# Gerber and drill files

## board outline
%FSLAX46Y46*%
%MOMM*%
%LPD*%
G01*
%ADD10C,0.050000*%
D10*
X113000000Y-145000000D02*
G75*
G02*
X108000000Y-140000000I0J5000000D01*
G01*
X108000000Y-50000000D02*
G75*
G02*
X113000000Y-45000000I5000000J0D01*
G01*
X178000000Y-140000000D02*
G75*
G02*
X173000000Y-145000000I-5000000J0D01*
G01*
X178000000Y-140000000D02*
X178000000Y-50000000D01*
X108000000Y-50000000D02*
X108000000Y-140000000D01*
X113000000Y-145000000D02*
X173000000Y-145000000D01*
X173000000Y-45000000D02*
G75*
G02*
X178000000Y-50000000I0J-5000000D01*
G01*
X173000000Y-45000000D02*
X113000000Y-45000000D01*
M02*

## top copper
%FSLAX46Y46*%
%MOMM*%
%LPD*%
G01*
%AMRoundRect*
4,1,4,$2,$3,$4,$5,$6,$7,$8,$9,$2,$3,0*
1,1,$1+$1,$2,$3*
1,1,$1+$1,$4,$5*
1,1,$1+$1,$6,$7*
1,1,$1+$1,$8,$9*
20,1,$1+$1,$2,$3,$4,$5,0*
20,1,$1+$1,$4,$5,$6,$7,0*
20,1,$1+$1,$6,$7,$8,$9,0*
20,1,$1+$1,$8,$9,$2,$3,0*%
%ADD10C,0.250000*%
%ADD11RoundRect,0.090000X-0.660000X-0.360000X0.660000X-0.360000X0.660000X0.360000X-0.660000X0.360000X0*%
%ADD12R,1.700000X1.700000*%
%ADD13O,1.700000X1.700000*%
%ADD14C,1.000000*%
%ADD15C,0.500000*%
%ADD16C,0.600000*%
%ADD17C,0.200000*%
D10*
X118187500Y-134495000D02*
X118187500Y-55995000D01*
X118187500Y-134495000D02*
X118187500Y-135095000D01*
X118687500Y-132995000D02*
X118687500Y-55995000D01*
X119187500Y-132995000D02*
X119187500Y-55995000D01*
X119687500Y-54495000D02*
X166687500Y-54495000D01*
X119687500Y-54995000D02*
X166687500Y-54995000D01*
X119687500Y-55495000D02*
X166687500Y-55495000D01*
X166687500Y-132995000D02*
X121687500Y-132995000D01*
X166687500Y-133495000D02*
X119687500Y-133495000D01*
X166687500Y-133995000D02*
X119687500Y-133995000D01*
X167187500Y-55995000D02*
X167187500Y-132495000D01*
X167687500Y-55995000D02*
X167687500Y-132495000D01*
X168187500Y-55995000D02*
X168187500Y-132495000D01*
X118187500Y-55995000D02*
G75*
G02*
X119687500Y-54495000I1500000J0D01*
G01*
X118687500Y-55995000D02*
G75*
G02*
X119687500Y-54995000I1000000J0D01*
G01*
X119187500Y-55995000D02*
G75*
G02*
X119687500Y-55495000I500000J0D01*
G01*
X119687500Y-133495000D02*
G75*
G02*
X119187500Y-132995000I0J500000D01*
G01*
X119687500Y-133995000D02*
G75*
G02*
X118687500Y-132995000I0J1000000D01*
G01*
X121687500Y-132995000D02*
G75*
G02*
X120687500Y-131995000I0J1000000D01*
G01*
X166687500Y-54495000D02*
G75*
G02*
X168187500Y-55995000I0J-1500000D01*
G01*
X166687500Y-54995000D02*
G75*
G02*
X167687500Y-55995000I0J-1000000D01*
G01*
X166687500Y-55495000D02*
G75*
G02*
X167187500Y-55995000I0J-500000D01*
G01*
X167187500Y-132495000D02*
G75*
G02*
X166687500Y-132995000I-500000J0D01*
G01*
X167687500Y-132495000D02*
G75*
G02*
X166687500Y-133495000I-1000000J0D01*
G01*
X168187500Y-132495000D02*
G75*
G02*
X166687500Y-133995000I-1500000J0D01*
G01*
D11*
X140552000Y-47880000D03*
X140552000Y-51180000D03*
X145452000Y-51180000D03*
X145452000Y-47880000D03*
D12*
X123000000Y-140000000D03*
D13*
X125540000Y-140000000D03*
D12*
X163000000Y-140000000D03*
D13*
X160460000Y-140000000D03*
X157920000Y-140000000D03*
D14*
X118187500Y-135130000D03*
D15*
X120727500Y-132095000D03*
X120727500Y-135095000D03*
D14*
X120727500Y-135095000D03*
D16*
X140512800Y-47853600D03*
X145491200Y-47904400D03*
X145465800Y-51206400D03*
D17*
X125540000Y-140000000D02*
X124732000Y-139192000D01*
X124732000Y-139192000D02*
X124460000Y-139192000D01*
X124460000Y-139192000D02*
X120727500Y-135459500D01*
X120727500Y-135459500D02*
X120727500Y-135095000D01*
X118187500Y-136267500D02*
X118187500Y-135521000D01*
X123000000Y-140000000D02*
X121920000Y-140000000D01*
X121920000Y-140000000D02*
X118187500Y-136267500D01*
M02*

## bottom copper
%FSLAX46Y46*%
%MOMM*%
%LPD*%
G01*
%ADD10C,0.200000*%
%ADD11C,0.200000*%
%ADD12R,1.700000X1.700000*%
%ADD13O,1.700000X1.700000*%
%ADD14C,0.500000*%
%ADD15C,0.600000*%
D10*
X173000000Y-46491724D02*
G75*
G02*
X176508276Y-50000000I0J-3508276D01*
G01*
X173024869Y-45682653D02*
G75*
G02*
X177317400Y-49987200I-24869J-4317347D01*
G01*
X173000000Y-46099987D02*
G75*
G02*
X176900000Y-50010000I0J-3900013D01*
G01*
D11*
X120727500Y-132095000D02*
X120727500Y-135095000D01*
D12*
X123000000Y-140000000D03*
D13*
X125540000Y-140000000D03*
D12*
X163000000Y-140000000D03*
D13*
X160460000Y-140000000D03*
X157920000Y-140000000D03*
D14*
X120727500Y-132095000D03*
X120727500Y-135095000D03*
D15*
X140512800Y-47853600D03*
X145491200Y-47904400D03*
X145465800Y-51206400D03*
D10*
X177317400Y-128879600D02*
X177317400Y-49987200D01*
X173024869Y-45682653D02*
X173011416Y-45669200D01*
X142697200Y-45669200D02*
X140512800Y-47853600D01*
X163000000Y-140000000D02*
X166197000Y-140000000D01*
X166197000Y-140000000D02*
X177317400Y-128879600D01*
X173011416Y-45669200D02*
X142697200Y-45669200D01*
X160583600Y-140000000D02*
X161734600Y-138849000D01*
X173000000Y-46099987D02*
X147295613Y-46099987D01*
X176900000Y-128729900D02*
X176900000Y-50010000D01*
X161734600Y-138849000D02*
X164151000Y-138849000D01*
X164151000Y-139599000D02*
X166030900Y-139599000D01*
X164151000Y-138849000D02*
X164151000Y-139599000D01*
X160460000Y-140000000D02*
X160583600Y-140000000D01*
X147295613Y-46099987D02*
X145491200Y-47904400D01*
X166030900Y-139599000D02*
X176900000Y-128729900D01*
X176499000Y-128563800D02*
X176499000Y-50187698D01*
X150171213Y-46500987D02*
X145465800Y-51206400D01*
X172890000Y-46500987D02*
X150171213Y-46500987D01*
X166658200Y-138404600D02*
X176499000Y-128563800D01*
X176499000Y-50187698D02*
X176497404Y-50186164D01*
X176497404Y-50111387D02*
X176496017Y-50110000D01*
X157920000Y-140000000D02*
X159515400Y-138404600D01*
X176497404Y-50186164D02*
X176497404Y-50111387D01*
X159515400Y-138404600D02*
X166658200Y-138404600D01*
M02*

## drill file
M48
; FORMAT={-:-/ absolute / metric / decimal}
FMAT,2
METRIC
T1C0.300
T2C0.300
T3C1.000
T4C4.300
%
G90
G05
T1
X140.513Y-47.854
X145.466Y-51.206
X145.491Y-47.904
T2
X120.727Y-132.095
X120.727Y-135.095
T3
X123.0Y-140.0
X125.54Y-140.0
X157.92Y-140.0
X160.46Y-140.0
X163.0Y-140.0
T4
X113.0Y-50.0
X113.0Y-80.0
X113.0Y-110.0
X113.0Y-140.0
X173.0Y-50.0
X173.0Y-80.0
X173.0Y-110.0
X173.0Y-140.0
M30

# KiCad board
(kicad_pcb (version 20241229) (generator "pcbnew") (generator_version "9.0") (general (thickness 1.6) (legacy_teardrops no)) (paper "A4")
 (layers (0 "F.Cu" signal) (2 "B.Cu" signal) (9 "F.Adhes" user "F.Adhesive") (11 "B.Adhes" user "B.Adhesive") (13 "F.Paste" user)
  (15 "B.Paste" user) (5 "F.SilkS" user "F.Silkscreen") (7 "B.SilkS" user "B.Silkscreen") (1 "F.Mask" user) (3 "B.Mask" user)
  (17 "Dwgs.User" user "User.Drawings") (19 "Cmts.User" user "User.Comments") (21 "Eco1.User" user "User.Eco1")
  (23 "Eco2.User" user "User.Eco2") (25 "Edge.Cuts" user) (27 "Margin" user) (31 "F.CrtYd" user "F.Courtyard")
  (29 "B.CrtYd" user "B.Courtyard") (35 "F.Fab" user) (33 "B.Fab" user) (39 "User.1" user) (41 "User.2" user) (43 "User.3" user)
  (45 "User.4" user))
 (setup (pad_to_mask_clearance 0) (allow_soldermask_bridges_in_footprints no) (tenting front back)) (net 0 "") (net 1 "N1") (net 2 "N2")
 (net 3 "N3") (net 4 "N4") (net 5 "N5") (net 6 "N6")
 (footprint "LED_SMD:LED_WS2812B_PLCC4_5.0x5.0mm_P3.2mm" (layer "F.Cu") (at 143.002 49.53)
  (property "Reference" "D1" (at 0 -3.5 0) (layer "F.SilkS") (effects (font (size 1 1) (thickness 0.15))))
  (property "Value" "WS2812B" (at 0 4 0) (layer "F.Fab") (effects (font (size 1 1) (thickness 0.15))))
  (pad "1" smd roundrect (at -2.45 -1.65) (size 1.5 0.9) (layers "F.Cu" "F.Mask" "F.Paste") (roundrect_rratio 0.1) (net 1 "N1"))
  (pad "2" smd roundrect (at -2.45 1.65) (size 1.5 0.9) (layers "F.Cu" "F.Mask" "F.Paste") (roundrect_rratio 0.1) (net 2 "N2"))
  (pad "3" smd roundrect (at 2.45 1.65) (size 1.5 0.9) (layers "F.Cu" "F.Mask" "F.Paste") (roundrect_rratio 0.1) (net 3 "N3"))
  (pad "4" smd roundrect (at 2.45 -1.65) (size 1.5 0.9) (layers "F.Cu" "F.Mask" "F.Paste") (roundrect_rratio 0.1) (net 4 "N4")))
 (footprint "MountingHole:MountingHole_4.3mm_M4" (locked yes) (layer "F.Cu") (at 113 50)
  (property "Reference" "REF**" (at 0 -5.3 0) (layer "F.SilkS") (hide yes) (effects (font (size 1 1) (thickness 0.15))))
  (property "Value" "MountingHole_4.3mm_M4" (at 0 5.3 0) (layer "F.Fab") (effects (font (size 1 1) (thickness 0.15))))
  (pad "" np_thru_hole circle (at 0 0) (size 4.3 4.3) (drill 4.3) (layers "*.Cu" "*.Mask")))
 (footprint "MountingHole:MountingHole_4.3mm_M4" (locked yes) (layer "F.Cu") (at 173 50)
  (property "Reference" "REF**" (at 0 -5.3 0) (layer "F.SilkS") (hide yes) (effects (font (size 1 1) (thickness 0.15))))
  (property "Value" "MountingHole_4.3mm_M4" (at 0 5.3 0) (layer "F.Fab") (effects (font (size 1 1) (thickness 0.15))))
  (pad "" np_thru_hole circle (at 0 0) (size 4.3 4.3) (drill 4.3) (layers "*.Cu" "*.Mask")))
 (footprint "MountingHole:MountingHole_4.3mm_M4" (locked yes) (layer "F.Cu") (at 173 80)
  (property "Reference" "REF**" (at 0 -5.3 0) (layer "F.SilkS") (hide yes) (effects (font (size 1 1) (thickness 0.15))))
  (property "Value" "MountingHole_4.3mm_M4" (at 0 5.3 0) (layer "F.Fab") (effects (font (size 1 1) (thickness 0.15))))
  (pad "" np_thru_hole circle (at 0 0) (size 4.3 4.3) (drill 4.3) (layers "*.Cu" "*.Mask")))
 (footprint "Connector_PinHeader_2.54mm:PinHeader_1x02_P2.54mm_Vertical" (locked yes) (layer "F.Cu") (at 123 140 90)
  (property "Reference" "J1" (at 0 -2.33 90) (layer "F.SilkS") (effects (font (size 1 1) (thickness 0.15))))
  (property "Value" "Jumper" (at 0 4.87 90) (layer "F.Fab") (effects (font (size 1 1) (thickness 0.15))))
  (pad "1" thru_hole rect (at 0 0 90) (size 1.7 1.7) (drill 1) (layers "*.Cu" "*.Mask") (remove_unused_layers no) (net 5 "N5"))
  (pad "2" thru_hole oval (at 0 2.54 90) (size 1.7 1.7) (drill 1) (layers "*.Cu" "*.Mask") (remove_unused_layers no) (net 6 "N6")))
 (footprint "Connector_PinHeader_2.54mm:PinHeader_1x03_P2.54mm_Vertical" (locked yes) (layer "F.Cu") (at 163 140 -90)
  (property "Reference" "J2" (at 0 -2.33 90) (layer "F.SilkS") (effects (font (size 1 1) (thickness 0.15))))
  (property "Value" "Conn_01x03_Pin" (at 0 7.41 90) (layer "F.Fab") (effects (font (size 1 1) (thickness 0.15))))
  (pad "1" thru_hole rect (at 0 0 270) (size 1.7 1.7) (drill 1) (layers "*.Cu" "*.Mask") (remove_unused_layers no) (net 1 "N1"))
  (pad "2" thru_hole oval (at 0 2.54 270) (size 1.7 1.7) (drill 1) (layers "*.Cu" "*.Mask") (remove_unused_layers no) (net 4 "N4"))
  (pad "3" thru_hole oval (at 0 5.08 270) (size 1.7 1.7) (drill 1) (layers "*.Cu" "*.Mask") (remove_unused_layers no) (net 3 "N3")))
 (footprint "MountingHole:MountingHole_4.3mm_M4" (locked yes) (layer "F.Cu") (at 113 140)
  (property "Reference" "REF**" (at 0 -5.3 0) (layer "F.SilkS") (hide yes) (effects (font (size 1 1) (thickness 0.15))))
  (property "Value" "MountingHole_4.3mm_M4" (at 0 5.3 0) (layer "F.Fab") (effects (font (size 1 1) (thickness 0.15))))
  (pad "" np_thru_hole circle (at 0 0) (size 4.3 4.3) (drill 4.3) (layers "*.Cu" "*.Mask")))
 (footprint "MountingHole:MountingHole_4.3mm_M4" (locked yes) (layer "F.Cu") (at 173 140)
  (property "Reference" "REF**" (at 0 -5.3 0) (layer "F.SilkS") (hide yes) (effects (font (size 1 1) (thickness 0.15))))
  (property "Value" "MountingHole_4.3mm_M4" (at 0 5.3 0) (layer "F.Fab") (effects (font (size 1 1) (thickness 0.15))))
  (pad "" np_thru_hole circle (at 0 0) (size 4.3 4.3) (drill 4.3) (layers "*.Cu" "*.Mask")))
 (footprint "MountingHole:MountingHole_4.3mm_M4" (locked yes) (layer "F.Cu") (at 173 110)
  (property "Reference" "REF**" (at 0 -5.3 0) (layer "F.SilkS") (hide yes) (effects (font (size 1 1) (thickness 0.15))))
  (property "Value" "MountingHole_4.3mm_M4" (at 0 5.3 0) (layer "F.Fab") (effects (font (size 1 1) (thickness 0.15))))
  (pad "" np_thru_hole circle (at 0 0) (size 4.3 4.3) (drill 4.3) (layers "*.Cu" "*.Mask")))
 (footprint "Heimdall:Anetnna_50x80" (layer "F.Cu") (at 118.1875 134.495)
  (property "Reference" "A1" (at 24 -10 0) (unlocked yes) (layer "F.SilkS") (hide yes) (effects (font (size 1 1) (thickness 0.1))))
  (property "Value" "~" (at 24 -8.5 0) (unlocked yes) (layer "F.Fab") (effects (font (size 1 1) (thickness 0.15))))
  (fp_line (start 0 0) (end 0 -78.5) (stroke (width 0.25) (type solid)) (layer "F.Cu"))
  (fp_line (start 0 0) (end 0 0.6) (stroke (width 0.25) (type solid)) (layer "F.Cu"))
  (fp_line (start 0.5 -1.5) (end 0.5 -78.5) (stroke (width 0.25) (type solid)) (layer "F.Cu"))
  (fp_line (start 1 -1.5) (end 1 -78.5) (stroke (width 0.25) (type solid)) (layer "F.Cu"))
  (fp_line (start 1.5 -80) (end 48.5 -80) (stroke (width 0.25) (type solid)) (layer "F.Cu"))
  (fp_line (start 1.5 -79.5) (end 48.5 -79.5) (stroke (width 0.25) (type solid)) (layer "F.Cu"))
  (fp_line (start 1.5 -79) (end 48.5 -79) (stroke (width 0.25) (type solid)) (layer "F.Cu"))
  (fp_line (start 48.5 -1.5) (end 3.5 -1.5) (stroke (width 0.25) (type solid)) (layer "F.Cu"))
  (fp_line (start 48.5 -1) (end 1.5 -1) (stroke (width 0.25) (type solid)) (layer "F.Cu"))
  (fp_line (start 48.5 -0.5) (end 1.5 -0.5) (stroke (width 0.25) (type solid)) (layer "F.Cu"))
  (fp_line (start 49 -78.5) (end 49 -2) (stroke (width 0.25) (type solid)) (layer "F.Cu"))
  (fp_line (start 49.5 -78.5) (end 49.5 -2) (stroke (width 0.25) (type solid)) (layer "F.Cu"))
  (fp_line (start 50 -78.5) (end 50 -2) (stroke (width 0.25) (type solid)) (layer "F.Cu"))
  (fp_arc (start 0 -78.5) (mid 0.43934 -79.56066) (end 1.5 -80) (stroke (width 0.25) (type solid)) (layer "F.Cu"))
  (fp_arc (start 0.5 -78.5) (mid 0.792893 -79.207107) (end 1.5 -79.5) (stroke (width 0.25) (type solid)) (layer "F.Cu"))
  (fp_arc (start 1 -78.5) (mid 1.146447 -78.853553) (end 1.5 -79) (stroke (width 0.25) (type solid)) (layer "F.Cu"))
  (fp_arc (start 1.5 -1) (mid 1.146447 -1.146447) (end 1 -1.5) (stroke (width 0.25) (type solid)) (layer "F.Cu"))
  (fp_arc (start 1.5 -0.5) (mid 0.792893 -0.792893) (end 0.5 -1.5) (stroke (width 0.25) (type solid)) (layer "F.Cu"))
  (fp_arc (start 3.5 -1.5) (mid 2.792893 -1.792893) (end 2.5 -2.5) (stroke (width 0.25) (type solid)) (layer "F.Cu"))
  (fp_arc (start 48.5 -80) (mid 49.56066 -79.56066) (end 50 -78.5) (stroke (width 0.25) (type solid)) (layer "F.Cu"))
  (fp_arc (start 48.5 -79.5) (mid 49.207107 -79.207107) (end 49.5 -78.5) (stroke (width 0.25) (type solid)) (layer "F.Cu"))
  (fp_arc (start 48.5 -79) (mid 48.853553 -78.853553) (end 49 -78.5) (stroke (width 0.25) (type solid)) (layer "F.Cu"))
  (fp_arc (start 49 -2) (mid 48.853553 -1.646447) (end 48.5 -1.5) (stroke (width 0.25) (type solid)) (layer "F.Cu"))
  (fp_arc (start 49.5 -2) (mid 49.207107 -1.292893) (end 48.5 -1) (stroke (width 0.25) (type solid)) (layer "F.Cu"))
  (fp_arc (start 50 -2) (mid 49.56066 -0.93934) (end 48.5 -0.5) (stroke (width 0.25) (type solid)) (layer "F.Cu"))
  (fp_line (start 2.54 -2.4) (end 2.54 0.6) (stroke (width 0.2) (type default)) (layer "B.Cu"))
  (pad "1" smd circle (at 0 0.635) (size 1 1) (layers "F.Cu") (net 5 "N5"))
  (pad "2" thru_hole circle (at 2.54 -2.4) (size 0.5 0.5) (drill 0.3) (layers "*.Cu" "*.Mask") (remove_unused_layers no) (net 6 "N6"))
  (pad "2" thru_hole circle (at 2.54 0.6) (size 0.5 0.5) (drill 0.3) (layers "*.Cu" "*.Mask") (remove_unused_layers no) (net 6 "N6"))
  (pad "2" smd circle (at 2.54 0.6) (size 1 1) (layers "F.Cu") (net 6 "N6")))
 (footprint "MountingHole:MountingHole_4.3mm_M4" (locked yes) (layer "F.Cu") (at 113 110)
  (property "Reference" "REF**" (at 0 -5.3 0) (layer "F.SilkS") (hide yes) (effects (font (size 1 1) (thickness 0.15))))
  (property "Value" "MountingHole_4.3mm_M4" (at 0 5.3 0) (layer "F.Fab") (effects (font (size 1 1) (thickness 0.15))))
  (pad "" np_thru_hole circle (at 0 0) (size 4.3 4.3) (drill 4.3) (layers "*.Cu" "*.Mask")))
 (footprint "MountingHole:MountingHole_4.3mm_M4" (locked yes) (layer "F.Cu") (at 113 80)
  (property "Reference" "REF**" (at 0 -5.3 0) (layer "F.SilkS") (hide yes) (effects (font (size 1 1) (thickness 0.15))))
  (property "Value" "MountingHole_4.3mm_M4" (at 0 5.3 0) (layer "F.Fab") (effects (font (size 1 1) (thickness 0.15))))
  (pad "" np_thru_hole circle (at 0 0) (size 4.3 4.3) (drill 4.3) (layers "*.Cu" "*.Mask")))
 (gr_arc (start 173 46.491724) (mid 175.480726 47.519274) (end 176.508276 50) (stroke (width 0.2) (type default)) (layer "B.Cu") (net 3))
 (gr_arc (start 173.024869 45.682653) (mid 176.05714 46.951394) (end 177.3174 49.9872) (stroke (width 0.2) (type default)) (layer "B.Cu")
  (net 1))
 (gr_arc (start 173 46.099987) (mid 175.761259 47.245812) (end 176.9 50.01) (stroke (width 0.2) (type default)) (layer "B.Cu") (net 4))
 (gr_arc (start 113 145) (mid 109.464466 143.535534) (end 108 140) (stroke (width 0.05) (type default)) (layer "Edge.Cuts"))
 (gr_arc (start 108 50) (mid 109.464466 46.464466) (end 113 45) (stroke (width 0.05) (type default)) (layer "Edge.Cuts"))
 (gr_arc (start 178 140) (mid 176.535534 143.535534) (end 173 145) (stroke (width 0.05) (type default)) (layer "Edge.Cuts"))
 (gr_line (start 178 140) (end 178 50) (stroke (width 0.05) (type default)) (layer "Edge.Cuts"))
 (gr_line (start 108 50) (end 108 140) (stroke (width 0.05) (type default)) (layer "Edge.Cuts"))
 (gr_line (start 113 145) (end 173 145) (stroke (width 0.05) (type default)) (layer "Edge.Cuts"))
 (gr_arc (start 173 45) (mid 176.535534 46.464466) (end 178 50) (stroke (width 0.05) (type default)) (layer "Edge.Cuts"))
 (gr_line (start 173 45) (end 113 45) (stroke (width 0.05) (type default)) (layer "Edge.Cuts"))
 (segment (start 125.54 140) (end 124.732 139.192) (width 0.2) (layer "F.Cu") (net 6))
 (segment (start 124.732 139.192) (end 124.46 139.192) (width 0.2) (layer "F.Cu") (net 6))
 (segment (start 124.46 139.192) (end 120.7275 135.4595) (width 0.2) (layer "F.Cu") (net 6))
 (segment (start 120.7275 135.4595) (end 120.7275 135.095) (width 0.2) (layer "F.Cu") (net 6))
 (segment (start 118.1875 136.2675) (end 118.1875 135.521) (width 0.2) (layer "F.Cu") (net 5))
 (segment (start 123 140) (end 121.92 140) (width 0.2) (layer "F.Cu") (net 5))
 (segment (start 121.92 140) (end 118.1875 136.2675) (width 0.2) (layer "F.Cu") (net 5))
 (via (at 140.5128 47.8536) (size 0.6) (drill 0.3) (layers "F.Cu" "B.Cu") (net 1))
 (segment (start 177.3174 128.8796) (end 177.3174 49.9872) (width 0.2) (layer "B.Cu") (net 1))
 (segment (start 173.024869 45.682653) (end 173.011416 45.6692) (width 0.2) (layer "B.Cu") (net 1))
 (segment (start 142.6972 45.6692) (end 140.5128 47.8536) (width 0.2) (layer "B.Cu") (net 1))
 (segment (start 163 140) (end 166.197 140) (width 0.2) (layer "B.Cu") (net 1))
 (segment (start 166.197 140) (end 177.3174 128.8796) (width 0.2) (layer "B.Cu") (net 1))
 (segment (start 173.011416 45.6692) (end 142.6972 45.6692) (width 0.2) (layer "B.Cu") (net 1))
 (via (at 145.4912 47.9044) (size 0.6) (drill 0.3) (layers "F.Cu" "B.Cu") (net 4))
 (segment (start 160.5836 140) (end 161.7346 138.849) (width 0.2) (layer "B.Cu") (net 4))
 (segment (start 173 46.099987) (end 147.295613 46.099987) (width 0.2) (layer "B.Cu") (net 4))
 (segment (start 176.9 128.7299) (end 176.9 50.01) (width 0.2) (layer "B.Cu") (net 4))
 (segment (start 161.7346 138.849) (end 164.151 138.849) (width 0.2) (layer "B.Cu") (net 4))
 (segment (start 164.151 139.599) (end 166.0309 139.599) (width 0.2) (layer "B.Cu") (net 4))
 (segment (start 164.151 138.849) (end 164.151 139.599) (width 0.2) (layer "B.Cu") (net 4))
 (segment (start 160.46 140) (end 160.5836 140) (width 0.2) (layer "B.Cu") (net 4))
 (segment (start 147.295613 46.099987) (end 145.4912 47.9044) (width 0.2) (layer "B.Cu") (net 4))
 (segment (start 166.0309 139.599) (end 176.9 128.7299) (width 0.2) (layer "B.Cu") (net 4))
 (via (at 145.4658 51.2064) (size 0.6) (drill 0.3) (layers "F.Cu" "B.Cu") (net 3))
 (segment (start 176.499 128.5638) (end 176.499 50.187698) (width 0.2) (layer "B.Cu") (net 3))
 (segment (start 150.171213 46.500987) (end 145.4658 51.2064) (width 0.2) (layer "B.Cu") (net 3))
 (segment (start 172.89 46.500987) (end 150.171213 46.500987) (width 0.2) (layer "B.Cu") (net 3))
 (segment (start 166.6582 138.4046) (end 176.499 128.5638) (width 0.2) (layer "B.Cu") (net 3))
 (segment (start 176.499 50.187698) (end 176.497404 50.186164) (width 0.2) (layer "B.Cu") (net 3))
 (segment (start 176.497404 50.111387) (end 176.496017 50.11) (width 0.2) (layer "B.Cu") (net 3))
 (segment (start 157.92 140) (end 159.5154 138.4046) (width 0.2) (layer "B.Cu") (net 3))
 (segment (start 176.497404 50.186164) (end 176.497404 50.111387) (width 0.2) (layer "B.Cu") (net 3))
 (segment (start 159.5154 138.4046) (end 166.6582 138.4046) (width 0.2) (layer "B.Cu") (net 3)))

